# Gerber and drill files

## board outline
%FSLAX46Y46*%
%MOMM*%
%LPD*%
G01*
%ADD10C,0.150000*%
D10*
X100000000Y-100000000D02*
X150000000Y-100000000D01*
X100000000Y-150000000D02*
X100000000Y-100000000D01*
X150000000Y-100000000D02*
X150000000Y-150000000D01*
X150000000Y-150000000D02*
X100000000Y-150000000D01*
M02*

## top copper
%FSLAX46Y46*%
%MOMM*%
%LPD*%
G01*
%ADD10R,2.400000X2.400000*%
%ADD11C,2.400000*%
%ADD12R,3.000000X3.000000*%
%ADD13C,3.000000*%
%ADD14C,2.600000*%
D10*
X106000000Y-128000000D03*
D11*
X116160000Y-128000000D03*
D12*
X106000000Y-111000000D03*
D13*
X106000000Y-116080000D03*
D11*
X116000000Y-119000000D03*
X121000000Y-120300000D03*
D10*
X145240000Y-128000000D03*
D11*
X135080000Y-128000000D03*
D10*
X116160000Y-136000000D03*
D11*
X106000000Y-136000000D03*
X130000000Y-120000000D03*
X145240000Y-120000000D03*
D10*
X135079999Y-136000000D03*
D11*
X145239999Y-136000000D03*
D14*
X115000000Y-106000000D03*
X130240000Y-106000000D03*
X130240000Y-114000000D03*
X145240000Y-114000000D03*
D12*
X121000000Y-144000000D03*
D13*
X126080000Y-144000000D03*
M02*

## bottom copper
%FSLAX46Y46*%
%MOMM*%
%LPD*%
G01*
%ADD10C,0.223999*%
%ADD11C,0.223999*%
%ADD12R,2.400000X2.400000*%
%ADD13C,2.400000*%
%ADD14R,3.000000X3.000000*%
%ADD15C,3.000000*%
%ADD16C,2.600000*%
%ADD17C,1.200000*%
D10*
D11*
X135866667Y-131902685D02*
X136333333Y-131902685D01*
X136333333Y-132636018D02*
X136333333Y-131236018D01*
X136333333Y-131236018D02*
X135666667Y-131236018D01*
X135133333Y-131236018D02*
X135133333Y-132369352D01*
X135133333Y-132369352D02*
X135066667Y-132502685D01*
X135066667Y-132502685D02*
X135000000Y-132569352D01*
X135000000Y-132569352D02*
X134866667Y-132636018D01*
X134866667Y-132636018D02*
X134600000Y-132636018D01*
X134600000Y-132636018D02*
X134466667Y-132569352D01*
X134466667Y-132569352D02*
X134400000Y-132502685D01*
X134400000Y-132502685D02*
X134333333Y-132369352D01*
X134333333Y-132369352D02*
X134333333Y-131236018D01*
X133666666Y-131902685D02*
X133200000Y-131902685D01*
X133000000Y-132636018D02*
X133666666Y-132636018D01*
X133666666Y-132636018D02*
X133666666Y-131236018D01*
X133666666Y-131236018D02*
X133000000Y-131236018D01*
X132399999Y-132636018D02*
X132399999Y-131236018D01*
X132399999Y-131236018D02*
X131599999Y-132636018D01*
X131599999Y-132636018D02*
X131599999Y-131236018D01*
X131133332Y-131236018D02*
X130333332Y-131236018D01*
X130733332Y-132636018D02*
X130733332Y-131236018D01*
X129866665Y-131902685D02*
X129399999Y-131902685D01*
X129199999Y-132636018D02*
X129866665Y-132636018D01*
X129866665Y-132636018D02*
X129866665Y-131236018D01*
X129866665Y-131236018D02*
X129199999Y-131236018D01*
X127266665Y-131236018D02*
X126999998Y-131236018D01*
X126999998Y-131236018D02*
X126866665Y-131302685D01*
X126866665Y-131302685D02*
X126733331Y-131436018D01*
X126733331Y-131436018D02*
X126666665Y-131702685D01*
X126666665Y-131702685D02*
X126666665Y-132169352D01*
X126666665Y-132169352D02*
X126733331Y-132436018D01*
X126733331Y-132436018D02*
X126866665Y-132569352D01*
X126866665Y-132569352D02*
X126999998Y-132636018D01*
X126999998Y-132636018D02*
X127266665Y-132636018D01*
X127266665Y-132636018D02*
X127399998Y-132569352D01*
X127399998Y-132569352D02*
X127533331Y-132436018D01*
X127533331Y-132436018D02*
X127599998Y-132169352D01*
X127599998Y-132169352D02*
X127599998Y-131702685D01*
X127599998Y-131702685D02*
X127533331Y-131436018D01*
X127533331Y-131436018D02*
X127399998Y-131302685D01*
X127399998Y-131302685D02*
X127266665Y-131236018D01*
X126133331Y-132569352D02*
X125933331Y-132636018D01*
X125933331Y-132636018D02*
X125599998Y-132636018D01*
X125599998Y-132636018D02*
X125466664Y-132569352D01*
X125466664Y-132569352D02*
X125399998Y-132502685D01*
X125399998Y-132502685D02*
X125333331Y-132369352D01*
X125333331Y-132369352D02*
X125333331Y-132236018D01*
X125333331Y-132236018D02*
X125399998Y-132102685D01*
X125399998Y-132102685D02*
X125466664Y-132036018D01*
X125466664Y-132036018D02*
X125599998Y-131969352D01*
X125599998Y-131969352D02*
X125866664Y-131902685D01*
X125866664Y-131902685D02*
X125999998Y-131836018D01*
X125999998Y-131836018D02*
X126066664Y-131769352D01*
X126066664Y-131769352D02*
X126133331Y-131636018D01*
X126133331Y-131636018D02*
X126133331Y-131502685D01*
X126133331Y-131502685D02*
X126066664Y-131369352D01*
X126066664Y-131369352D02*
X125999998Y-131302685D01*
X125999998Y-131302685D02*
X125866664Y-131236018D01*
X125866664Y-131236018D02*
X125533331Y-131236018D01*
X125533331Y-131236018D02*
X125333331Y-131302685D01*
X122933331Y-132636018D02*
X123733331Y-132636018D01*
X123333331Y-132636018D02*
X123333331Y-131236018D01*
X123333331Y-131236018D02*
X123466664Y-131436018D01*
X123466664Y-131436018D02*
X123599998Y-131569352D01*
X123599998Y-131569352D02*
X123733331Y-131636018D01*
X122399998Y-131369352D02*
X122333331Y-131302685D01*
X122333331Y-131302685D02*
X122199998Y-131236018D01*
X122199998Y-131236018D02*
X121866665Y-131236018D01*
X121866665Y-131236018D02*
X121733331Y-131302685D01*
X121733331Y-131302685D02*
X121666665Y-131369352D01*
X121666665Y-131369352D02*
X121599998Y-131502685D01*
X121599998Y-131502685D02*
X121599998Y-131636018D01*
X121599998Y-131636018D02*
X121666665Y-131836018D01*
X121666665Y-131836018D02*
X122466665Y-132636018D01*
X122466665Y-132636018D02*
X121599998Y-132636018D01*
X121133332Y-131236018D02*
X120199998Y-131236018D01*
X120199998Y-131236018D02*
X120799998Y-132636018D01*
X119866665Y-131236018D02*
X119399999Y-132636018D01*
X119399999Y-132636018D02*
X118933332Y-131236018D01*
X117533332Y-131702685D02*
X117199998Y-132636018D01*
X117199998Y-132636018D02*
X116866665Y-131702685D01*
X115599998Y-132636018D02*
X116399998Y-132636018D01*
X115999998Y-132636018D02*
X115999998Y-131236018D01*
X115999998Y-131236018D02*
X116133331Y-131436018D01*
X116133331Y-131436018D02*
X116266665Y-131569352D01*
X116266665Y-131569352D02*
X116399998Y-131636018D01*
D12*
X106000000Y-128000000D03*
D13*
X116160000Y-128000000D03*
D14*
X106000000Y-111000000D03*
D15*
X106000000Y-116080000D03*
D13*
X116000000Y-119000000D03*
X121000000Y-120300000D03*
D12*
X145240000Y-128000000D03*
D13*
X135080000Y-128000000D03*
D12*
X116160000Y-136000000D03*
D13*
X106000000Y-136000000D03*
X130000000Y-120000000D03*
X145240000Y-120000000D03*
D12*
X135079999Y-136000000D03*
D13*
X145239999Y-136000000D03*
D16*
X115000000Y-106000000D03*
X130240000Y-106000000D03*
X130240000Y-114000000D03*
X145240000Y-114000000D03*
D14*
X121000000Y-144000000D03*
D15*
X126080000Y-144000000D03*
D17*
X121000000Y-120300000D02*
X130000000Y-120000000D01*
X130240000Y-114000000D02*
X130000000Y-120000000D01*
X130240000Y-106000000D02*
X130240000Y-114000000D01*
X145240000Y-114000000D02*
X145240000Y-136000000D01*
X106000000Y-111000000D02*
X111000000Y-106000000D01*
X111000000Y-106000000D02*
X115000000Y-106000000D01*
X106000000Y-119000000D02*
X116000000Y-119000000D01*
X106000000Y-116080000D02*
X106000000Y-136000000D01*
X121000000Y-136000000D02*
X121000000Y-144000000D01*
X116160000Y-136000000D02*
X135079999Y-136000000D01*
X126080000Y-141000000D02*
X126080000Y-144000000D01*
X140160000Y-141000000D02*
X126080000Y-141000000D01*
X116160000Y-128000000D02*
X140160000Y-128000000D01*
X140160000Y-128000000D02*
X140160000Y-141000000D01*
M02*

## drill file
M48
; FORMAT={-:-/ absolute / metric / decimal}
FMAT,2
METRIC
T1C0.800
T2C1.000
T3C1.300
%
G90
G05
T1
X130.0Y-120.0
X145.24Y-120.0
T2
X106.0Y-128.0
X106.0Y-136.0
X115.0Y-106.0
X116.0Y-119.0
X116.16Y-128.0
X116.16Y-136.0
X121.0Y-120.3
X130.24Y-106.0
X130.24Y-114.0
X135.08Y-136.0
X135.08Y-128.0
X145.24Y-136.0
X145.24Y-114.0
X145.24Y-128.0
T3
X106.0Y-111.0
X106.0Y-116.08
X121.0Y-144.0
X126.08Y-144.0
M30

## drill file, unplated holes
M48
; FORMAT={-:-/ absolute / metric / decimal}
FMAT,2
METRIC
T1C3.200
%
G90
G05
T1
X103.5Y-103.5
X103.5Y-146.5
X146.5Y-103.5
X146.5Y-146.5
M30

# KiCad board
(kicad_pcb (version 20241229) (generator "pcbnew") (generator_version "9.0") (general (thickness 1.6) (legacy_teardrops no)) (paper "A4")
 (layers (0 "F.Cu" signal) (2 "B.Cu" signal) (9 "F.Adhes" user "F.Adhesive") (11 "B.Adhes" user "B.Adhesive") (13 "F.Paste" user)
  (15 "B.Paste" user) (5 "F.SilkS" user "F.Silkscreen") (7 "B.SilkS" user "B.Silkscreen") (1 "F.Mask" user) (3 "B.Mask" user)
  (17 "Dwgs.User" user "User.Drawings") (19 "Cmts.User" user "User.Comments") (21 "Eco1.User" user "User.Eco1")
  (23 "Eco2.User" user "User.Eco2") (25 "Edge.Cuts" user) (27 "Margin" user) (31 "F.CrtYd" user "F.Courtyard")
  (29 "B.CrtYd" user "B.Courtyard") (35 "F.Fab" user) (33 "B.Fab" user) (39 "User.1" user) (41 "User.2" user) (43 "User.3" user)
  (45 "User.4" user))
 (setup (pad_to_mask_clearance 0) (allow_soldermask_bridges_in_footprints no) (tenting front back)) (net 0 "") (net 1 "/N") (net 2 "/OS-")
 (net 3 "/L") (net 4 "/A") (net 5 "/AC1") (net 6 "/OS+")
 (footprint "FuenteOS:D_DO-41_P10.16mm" (layer "F.Cu") (at 106 128)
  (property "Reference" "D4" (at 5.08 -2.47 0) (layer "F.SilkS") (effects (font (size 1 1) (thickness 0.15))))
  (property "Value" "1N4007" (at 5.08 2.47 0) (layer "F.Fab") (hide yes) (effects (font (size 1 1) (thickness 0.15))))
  (pad "1" thru_hole rect (at 0 0) (size 2.4 2.4) (drill 1) (layers "B.Cu" "B.Mask") (remove_unused_layers no) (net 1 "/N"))
  (pad "2" thru_hole circle (at 10.16 0) (size 2.4 2.4) (drill 1) (layers "B.Cu" "B.Mask") (remove_unused_layers no) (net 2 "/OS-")))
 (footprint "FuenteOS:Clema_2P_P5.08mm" (layer "F.Cu") (at 106 111 -90)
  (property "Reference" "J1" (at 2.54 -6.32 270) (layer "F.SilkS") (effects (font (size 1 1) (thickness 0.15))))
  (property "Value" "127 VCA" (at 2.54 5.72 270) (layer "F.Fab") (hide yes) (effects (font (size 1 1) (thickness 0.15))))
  (pad "1" thru_hole rect (at 0 0 270) (size 3 3) (drill 1.3) (layers "B.Cu" "B.Mask") (remove_unused_layers no) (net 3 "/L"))
  (pad "2" thru_hole circle (at 5.08 0 270) (size 3 3) (drill 1.3) (layers "B.Cu" "B.Mask") (remove_unused_layers no) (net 1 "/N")))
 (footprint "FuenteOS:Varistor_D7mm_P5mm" (layer "F.Cu") (at 116 119)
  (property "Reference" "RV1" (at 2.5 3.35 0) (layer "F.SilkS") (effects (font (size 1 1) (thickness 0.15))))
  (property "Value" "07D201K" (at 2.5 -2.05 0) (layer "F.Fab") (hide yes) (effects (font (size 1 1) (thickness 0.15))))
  (pad "1" thru_hole circle (at 0 0) (size 2.4 2.4) (drill 1) (layers "B.Cu" "B.Mask") (remove_unused_layers no) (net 1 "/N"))
  (pad "2" thru_hole circle (at 5 1.3) (size 2.4 2.4) (drill 1) (layers "B.Cu" "B.Mask") (remove_unused_layers no) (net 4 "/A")))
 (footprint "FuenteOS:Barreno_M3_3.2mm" (layer "F.Cu") (at 146.5 146.5)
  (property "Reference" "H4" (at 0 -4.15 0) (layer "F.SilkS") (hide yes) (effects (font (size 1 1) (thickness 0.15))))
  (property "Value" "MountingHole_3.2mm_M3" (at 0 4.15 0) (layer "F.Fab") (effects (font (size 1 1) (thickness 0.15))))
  (pad "" np_thru_hole circle (at 0 0) (size 3.2 3.2) (drill 3.2) (layers "*.Cu" "*.Mask")))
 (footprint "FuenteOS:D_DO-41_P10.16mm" (layer "F.Cu") (at 145.24 128 180)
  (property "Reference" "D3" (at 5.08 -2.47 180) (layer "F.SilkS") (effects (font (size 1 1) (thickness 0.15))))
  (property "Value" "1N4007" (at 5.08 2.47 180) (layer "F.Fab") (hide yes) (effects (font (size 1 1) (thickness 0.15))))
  (pad "1" thru_hole rect (at 0 0 180) (size 2.4 2.4) (drill 1) (layers "B.Cu" "B.Mask") (remove_unused_layers no) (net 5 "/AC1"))
  (pad "2" thru_hole circle (at 10.16 0 180) (size 2.4 2.4) (drill 1) (layers "B.Cu" "B.Mask") (remove_unused_layers no) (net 2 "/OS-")))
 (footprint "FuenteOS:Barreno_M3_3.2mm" (layer "F.Cu") (at 103.5 146.5)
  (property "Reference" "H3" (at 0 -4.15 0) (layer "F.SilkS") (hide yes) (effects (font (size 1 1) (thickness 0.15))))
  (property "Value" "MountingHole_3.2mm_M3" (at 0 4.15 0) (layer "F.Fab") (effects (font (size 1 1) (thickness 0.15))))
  (pad "" np_thru_hole circle (at 0 0) (size 3.2 3.2) (drill 3.2) (layers "*.Cu" "*.Mask")))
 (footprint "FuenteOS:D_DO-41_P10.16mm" (layer "F.Cu") (at 116.16 136 180)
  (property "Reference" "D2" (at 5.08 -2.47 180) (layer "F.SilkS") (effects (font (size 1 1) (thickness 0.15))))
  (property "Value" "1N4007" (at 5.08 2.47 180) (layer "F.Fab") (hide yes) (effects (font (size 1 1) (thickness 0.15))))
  (pad "1" thru_hole rect (at 0 0 180) (size 2.4 2.4) (drill 1) (layers "B.Cu" "B.Mask") (remove_unused_layers no) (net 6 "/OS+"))
  (pad "2" thru_hole circle (at 10.16 0 180) (size 2.4 2.4) (drill 1) (layers "B.Cu" "B.Mask") (remove_unused_layers no) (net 1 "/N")))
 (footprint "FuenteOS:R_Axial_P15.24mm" (layer "F.Cu") (at 130 120)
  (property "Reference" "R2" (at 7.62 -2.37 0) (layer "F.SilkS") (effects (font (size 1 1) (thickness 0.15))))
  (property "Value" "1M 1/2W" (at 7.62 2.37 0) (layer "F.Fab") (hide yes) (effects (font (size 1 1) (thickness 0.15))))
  (pad "1" thru_hole circle (at 0 0) (size 2.4 2.4) (drill 0.8) (layers "B.Cu" "B.Mask") (remove_unused_layers no) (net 4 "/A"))
  (pad "2" thru_hole circle (at 15.24 0) (size 2.4 2.4) (drill 0.8) (layers "B.Cu" "B.Mask") (remove_unused_layers no) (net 5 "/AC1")))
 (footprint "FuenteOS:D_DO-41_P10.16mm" (layer "F.Cu") (at 135.079999 136)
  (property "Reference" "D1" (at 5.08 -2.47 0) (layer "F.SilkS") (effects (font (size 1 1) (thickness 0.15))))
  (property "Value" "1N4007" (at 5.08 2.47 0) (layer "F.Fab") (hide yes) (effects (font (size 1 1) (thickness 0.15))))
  (pad "1" thru_hole rect (at 0 0) (size 2.4 2.4) (drill 1) (layers "B.Cu" "B.Mask") (remove_unused_layers no) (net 6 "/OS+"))
  (pad "2" thru_hole circle (at 10.16 0) (size 2.4 2.4) (drill 1) (layers "B.Cu" "B.Mask") (remove_unused_layers no) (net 5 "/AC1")))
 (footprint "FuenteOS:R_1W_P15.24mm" (layer "F.Cu") (at 115 106)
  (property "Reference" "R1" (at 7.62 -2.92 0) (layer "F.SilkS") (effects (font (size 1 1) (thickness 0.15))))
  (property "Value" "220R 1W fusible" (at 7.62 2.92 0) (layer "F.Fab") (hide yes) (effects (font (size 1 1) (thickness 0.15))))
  (pad "1" thru_hole circle (at 0 0) (size 2.6 2.6) (drill 1) (layers "B.Cu" "B.Mask") (remove_unused_layers no) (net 3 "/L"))
  (pad "2" thru_hole circle (at 15.24 0) (size 2.6 2.6) (drill 1) (layers "B.Cu" "B.Mask") (remove_unused_layers no) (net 4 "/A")))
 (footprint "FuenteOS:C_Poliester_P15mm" (layer "F.Cu") (at 130.24 114)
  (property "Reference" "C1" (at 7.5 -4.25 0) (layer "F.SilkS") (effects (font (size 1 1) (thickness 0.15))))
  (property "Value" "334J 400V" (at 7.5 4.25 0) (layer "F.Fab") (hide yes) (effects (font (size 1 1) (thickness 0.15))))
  (pad "1" thru_hole circle (at 0 0) (size 2.6 2.6) (drill 1) (layers "B.Cu" "B.Mask") (remove_unused_layers no) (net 4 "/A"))
  (pad "2" thru_hole circle (at 15 0) (size 2.6 2.6) (drill 1) (layers "B.Cu" "B.Mask") (remove_unused_layers no) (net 5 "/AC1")))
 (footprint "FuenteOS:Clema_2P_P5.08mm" (layer "F.Cu") (at 121 144)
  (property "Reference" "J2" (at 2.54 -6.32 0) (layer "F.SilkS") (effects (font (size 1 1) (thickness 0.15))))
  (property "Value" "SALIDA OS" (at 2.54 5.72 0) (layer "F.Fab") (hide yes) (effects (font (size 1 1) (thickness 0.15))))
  (pad "1" thru_hole rect (at 0 0) (size 3 3) (drill 1.3) (layers "B.Cu" "B.Mask") (remove_unused_layers no) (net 6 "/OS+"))
  (pad "2" thru_hole circle (at 5.08 0) (size 3 3) (drill 1.3) (layers "B.Cu" "B.Mask") (remove_unused_layers no) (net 2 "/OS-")))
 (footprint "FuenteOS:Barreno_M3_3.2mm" (layer "F.Cu") (at 146.5 103.5)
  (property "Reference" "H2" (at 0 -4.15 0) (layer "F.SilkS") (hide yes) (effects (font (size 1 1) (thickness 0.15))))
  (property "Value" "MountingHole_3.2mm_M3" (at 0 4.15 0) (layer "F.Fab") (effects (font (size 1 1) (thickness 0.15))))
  (pad "" np_thru_hole circle (at 0 0) (size 3.2 3.2) (drill 3.2) (layers "*.Cu" "*.Mask")))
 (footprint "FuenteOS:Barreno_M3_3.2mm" (layer "F.Cu") (at 103.5 103.5)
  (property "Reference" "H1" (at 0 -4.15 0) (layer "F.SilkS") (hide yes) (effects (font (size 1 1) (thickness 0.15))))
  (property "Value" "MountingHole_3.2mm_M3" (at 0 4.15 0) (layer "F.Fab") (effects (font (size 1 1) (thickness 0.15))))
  (pad "" np_thru_hole circle (at 0 0) (size 3.2 3.2) (drill 3.2) (layers "*.Cu" "*.Mask")))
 (gr_line (start 100 100) (end 150 100) (stroke (width 0.15) (type default)) (layer "Edge.Cuts"))
 (gr_line (start 100 150) (end 100 100) (stroke (width 0.15) (type default)) (layer "Edge.Cuts"))
 (gr_line (start 150 100) (end 150 150) (stroke (width 0.15) (type default)) (layer "Edge.Cuts"))
 (gr_line (start 150 150) (end 100 150) (stroke (width 0.15) (type default)) (layer "Edge.Cuts"))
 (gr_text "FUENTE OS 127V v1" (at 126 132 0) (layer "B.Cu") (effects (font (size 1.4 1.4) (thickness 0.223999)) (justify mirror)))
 (segment (start 121 120.3) (end 130 120) (width 1.2) (layer "B.Cu") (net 4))
 (segment (start 130.24 114) (end 130 120) (width 1.2) (layer "B.Cu") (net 4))
 (segment (start 130.24 106) (end 130.24 114) (width 1.2) (layer "B.Cu") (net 4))
 (segment (start 145.24 114) (end 145.24 136) (width 1.2) (layer "B.Cu") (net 5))
 (segment (start 106 111) (end 111 106) (width 1.2) (layer "B.Cu") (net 3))
 (segment (start 111 106) (end 115 106) (width 1.2) (layer "B.Cu") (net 3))
 (segment (start 106 119) (end 116 119) (width 1.2) (layer "B.Cu") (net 1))
 (segment (start 106 116.08) (end 106 136) (width 1.2) (layer "B.Cu") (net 1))
 (segment (start 121 136) (end 121 144) (width 1.2) (layer "B.Cu") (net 6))
 (segment (start 116.16 136) (end 135.079999 136) (width 1.2) (layer "B.Cu") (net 6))
 (segment (start 126.08 141) (end 126.08 144) (width 1.2) (layer "B.Cu") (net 2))
 (segment (start 140.16 141) (end 126.08 141) (width 1.2) (layer "B.Cu") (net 2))
 (segment (start 116.16 128) (end 140.16 128) (width 1.2) (layer "B.Cu") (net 2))
 (segment (start 140.16 128) (end 140.16 141) (width 1.2) (layer "B.Cu") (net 2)))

